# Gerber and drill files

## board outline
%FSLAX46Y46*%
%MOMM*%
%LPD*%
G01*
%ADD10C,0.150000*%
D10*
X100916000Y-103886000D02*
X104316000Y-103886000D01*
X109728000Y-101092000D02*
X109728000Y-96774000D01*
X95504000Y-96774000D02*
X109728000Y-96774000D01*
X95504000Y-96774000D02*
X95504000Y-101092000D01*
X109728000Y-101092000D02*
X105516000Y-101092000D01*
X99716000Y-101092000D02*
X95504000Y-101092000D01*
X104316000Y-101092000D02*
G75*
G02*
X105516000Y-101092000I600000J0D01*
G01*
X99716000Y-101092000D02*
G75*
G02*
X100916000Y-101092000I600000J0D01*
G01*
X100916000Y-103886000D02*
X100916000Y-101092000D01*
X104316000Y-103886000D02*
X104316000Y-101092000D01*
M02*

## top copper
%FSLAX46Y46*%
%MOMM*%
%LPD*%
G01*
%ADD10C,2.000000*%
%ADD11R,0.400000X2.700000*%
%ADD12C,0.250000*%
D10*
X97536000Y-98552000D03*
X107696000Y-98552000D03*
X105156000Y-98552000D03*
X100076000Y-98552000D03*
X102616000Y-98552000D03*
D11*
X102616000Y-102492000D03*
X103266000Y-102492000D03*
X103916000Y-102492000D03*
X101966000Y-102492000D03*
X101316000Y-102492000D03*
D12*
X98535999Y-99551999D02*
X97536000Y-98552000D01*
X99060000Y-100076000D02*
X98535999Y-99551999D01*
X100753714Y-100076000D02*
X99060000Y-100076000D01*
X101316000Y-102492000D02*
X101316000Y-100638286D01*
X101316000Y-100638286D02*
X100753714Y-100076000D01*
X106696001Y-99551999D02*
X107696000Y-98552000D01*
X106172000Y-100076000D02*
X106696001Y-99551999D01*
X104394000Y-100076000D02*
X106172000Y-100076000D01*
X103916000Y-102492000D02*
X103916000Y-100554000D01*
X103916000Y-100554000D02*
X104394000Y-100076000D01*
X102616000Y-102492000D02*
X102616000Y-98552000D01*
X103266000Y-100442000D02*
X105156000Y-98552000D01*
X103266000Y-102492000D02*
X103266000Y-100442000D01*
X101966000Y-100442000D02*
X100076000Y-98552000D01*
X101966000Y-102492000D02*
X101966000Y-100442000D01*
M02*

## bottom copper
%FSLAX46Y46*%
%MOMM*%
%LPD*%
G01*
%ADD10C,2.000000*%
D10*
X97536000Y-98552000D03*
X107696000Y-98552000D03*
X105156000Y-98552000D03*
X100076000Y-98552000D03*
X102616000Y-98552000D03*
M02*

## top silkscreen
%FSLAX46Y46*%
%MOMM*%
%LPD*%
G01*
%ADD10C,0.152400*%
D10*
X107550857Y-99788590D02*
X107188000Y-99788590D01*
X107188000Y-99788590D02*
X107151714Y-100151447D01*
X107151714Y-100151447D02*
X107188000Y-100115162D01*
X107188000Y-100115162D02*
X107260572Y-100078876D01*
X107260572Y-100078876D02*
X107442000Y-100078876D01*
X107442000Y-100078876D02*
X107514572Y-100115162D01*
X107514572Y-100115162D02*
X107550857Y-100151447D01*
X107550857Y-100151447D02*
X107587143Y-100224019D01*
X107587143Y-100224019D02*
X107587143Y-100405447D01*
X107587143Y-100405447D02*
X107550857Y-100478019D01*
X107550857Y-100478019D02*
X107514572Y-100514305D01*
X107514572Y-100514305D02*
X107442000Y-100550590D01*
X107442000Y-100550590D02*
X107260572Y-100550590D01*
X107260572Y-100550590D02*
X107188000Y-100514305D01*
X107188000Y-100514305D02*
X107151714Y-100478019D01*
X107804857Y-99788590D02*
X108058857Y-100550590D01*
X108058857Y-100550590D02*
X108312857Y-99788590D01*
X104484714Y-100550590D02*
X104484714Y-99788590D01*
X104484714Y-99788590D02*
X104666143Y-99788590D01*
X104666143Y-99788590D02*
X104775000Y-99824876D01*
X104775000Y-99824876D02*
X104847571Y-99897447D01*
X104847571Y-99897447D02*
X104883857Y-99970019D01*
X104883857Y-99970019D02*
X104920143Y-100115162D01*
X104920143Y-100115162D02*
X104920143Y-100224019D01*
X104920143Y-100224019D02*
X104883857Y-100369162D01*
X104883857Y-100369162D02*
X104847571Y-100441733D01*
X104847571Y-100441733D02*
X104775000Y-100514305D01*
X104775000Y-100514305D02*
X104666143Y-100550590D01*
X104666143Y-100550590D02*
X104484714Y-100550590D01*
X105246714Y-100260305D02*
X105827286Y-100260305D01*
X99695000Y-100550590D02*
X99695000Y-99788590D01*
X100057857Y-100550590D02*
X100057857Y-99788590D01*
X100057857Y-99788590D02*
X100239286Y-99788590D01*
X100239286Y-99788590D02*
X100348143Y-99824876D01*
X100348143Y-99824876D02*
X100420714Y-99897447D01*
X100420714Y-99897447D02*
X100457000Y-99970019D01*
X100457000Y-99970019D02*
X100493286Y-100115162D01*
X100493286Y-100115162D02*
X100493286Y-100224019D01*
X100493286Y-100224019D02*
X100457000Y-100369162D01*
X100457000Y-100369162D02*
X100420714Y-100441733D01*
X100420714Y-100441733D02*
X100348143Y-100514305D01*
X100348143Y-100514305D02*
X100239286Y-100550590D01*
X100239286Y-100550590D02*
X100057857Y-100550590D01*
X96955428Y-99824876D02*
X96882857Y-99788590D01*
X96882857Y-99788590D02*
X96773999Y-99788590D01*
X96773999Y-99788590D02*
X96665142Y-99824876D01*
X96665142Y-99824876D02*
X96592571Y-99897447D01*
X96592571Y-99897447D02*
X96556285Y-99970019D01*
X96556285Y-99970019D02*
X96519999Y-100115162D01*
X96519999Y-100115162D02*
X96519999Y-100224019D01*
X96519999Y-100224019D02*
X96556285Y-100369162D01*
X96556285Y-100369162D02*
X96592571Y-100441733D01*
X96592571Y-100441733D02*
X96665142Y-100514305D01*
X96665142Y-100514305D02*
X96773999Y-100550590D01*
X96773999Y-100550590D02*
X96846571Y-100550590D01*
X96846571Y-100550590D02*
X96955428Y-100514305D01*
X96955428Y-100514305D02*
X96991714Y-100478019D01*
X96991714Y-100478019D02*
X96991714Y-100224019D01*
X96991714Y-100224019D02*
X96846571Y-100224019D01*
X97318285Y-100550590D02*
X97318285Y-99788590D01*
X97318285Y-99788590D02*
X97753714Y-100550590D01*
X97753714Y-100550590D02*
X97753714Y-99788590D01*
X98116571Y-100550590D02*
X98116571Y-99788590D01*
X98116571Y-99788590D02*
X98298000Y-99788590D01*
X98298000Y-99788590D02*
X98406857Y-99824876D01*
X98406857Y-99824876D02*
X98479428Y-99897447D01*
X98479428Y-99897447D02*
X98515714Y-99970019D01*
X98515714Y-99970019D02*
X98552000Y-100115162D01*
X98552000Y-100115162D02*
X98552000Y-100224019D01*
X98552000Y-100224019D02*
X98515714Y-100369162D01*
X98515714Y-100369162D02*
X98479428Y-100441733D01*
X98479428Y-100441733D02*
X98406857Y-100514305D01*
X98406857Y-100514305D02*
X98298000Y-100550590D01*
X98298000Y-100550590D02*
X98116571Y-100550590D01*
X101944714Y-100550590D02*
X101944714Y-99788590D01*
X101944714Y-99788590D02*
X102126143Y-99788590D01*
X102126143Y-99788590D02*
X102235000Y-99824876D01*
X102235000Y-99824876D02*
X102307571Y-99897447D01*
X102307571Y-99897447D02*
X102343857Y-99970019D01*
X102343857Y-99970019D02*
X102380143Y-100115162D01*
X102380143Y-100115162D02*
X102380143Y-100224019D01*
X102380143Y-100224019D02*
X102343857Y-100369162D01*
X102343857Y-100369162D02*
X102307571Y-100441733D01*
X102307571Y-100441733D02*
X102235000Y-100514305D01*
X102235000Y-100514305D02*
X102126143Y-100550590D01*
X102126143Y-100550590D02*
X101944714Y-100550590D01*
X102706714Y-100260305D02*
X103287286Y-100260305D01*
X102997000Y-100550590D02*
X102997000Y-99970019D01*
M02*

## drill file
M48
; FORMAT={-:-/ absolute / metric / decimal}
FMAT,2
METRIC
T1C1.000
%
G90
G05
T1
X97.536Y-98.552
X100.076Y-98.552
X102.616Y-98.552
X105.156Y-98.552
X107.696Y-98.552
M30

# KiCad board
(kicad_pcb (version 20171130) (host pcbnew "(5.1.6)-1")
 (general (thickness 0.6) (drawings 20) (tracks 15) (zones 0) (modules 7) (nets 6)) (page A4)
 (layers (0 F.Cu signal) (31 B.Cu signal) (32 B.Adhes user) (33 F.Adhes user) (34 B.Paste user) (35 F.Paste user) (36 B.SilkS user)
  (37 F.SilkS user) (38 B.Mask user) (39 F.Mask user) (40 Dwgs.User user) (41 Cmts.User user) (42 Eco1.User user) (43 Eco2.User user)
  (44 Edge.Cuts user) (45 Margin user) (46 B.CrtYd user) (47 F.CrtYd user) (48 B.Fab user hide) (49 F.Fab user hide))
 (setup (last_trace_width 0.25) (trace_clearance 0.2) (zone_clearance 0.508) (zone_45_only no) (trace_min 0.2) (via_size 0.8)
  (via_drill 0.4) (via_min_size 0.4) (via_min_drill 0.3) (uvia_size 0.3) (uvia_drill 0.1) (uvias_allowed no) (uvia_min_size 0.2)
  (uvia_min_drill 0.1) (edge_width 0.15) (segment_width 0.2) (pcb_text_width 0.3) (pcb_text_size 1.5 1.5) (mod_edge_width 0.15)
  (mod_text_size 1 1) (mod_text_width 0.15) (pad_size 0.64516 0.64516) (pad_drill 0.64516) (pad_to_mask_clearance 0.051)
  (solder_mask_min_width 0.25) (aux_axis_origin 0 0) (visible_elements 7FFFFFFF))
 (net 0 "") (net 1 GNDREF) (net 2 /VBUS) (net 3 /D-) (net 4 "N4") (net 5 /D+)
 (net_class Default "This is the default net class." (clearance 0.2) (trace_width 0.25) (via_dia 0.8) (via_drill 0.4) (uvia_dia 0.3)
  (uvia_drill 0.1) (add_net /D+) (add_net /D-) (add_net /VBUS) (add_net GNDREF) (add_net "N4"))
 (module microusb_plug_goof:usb (layer B.Cu) (at 102.616 102.616)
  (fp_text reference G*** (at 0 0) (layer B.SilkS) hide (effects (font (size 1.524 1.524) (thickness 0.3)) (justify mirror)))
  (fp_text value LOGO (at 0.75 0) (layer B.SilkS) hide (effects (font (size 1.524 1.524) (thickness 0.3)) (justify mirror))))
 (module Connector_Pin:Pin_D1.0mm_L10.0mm (layer F.Cu) (at 97.536 98.552)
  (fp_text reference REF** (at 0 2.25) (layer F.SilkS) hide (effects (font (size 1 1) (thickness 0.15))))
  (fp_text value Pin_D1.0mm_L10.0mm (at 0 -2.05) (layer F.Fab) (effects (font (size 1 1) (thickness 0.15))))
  (pad 1 thru_hole circle (at 0 0) (size 2 2) (drill 1) (layers *.Cu *.Mask) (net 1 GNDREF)))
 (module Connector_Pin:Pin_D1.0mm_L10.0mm (layer F.Cu) (at 107.696 98.552)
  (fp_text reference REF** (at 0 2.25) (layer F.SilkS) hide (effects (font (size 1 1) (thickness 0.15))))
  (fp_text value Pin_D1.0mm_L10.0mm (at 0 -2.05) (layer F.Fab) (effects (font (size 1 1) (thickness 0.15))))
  (pad 1 thru_hole circle (at 0 0) (size 2 2) (drill 1) (layers *.Cu *.Mask) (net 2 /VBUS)))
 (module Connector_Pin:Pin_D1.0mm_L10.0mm (layer F.Cu) (at 105.156 98.552)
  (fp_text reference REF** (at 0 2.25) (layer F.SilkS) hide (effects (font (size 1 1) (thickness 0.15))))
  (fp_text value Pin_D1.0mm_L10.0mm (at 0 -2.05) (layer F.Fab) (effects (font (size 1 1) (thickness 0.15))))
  (pad 1 thru_hole circle (at 0 0) (size 2 2) (drill 1) (layers *.Cu *.Mask) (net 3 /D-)))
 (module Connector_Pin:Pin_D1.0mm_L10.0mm (layer F.Cu) (at 100.076 98.552)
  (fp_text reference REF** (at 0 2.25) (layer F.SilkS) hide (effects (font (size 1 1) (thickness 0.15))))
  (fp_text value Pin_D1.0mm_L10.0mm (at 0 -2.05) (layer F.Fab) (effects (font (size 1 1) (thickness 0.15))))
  (pad 1 thru_hole circle (at 0 0) (size 2 2) (drill 1) (layers *.Cu *.Mask) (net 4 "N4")))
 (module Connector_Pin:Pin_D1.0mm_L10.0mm (layer F.Cu) (at 102.616 98.552)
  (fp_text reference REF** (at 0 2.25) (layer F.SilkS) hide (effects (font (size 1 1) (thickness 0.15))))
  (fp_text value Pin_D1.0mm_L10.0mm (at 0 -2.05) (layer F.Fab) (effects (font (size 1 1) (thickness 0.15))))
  (pad 1 thru_hole circle (at 0 0) (size 2 2) (drill 1) (layers *.Cu *.Mask) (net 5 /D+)))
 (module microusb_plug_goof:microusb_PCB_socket (layer F.Cu) (at 102.616 102.492 180)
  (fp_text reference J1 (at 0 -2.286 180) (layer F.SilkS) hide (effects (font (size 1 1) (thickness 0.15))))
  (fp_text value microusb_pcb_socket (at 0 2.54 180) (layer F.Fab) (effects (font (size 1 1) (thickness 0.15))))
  (pad 3 smd rect (at 0 0 180) (size 0.4 2.7) (layers F.Cu F.Paste F.Mask) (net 5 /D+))
  (pad 2 smd rect (at -0.65 0 180) (size 0.4 2.7) (layers F.Cu F.Paste F.Mask) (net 3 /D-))
  (pad 1 smd rect (at -1.3 0 180) (size 0.4 2.7) (layers F.Cu F.Paste F.Mask) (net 2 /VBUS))
  (pad 4 smd rect (at 0.65 0 180) (size 0.4 2.7) (layers F.Cu F.Paste F.Mask) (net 4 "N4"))
  (pad 5 smd rect (at 1.3 0 180) (size 0.4 2.7) (layers F.Cu F.Paste F.Mask) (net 1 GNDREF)))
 (gr_line (start 100.916 103.886) (end 104.316 103.886) (layer Edge.Cuts) (width 0.15))
 (gr_line (start 109.728 101.092) (end 109.728 96.774) (layer Edge.Cuts) (width 0.15))
 (gr_line (start 95.504 96.774) (end 109.728 96.774) (layer Edge.Cuts) (width 0.15))
 (gr_line (start 95.504 96.774) (end 95.504 101.092) (layer Edge.Cuts) (width 0.15))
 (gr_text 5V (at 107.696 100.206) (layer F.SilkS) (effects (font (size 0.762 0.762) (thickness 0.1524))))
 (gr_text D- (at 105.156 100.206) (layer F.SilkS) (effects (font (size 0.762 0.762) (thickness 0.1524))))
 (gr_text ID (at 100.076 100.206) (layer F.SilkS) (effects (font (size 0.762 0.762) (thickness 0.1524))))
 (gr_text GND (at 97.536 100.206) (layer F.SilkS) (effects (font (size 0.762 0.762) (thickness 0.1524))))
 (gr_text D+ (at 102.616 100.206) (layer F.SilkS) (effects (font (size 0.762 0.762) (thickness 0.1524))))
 (gr_line (start 109.728 101.092) (end 105.516 101.092) (layer Edge.Cuts) (width 0.15))
 (gr_line (start 99.716 101.092) (end 95.504 101.092) (layer Edge.Cuts) (width 0.15))
 (gr_arc (start 104.916 101.092) (end 104.316 101.092) (angle 180) (layer Edge.Cuts) (width 0.15))
 (gr_arc (start 100.316 101.092) (end 100.916 101.092) (angle -180) (layer Edge.Cuts) (width 0.15))
 (gr_line (start 100.916 103.886) (end 100.916 101.092) (layer Edge.Cuts) (width 0.15))
 (gr_line (start 104.316 103.886) (end 104.316 101.092) (layer Edge.Cuts) (width 0.15))
 (segment (start 98.535999 99.551999) (end 97.536 98.552) (width 0.25) (layer F.Cu) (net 1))
 (segment (start 99.06 100.076) (end 98.535999 99.551999) (width 0.25) (layer F.Cu) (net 1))
 (segment (start 100.753714 100.076) (end 99.06 100.076) (width 0.25) (layer F.Cu) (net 1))
 (segment (start 101.316 102.492) (end 101.316 100.638286) (width 0.25) (layer F.Cu) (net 1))
 (segment (start 101.316 100.638286) (end 100.753714 100.076) (width 0.25) (layer F.Cu) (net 1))
 (segment (start 106.696001 99.551999) (end 107.696 98.552) (width 0.25) (layer F.Cu) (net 2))
 (segment (start 106.172 100.076) (end 106.696001 99.551999) (width 0.25) (layer F.Cu) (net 2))
 (segment (start 104.394 100.076) (end 106.172 100.076) (width 0.25) (layer F.Cu) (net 2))
 (segment (start 103.916 102.492) (end 103.916 100.554) (width 0.25) (layer F.Cu) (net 2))
 (segment (start 103.916 100.554) (end 104.394 100.076) (width 0.25) (layer F.Cu) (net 2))
 (segment (start 102.616 102.492) (end 102.616 98.552) (width 0.25) (layer F.Cu) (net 5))
 (segment (start 103.266 100.442) (end 105.156 98.552) (width 0.25) (layer F.Cu) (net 3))
 (segment (start 103.266 102.492) (end 103.266 100.442) (width 0.25) (layer F.Cu) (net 3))
 (segment (start 101.966 100.442) (end 100.076 98.552) (width 0.25) (layer F.Cu) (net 4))
 (segment (start 101.966 102.492) (end 101.966 100.442) (width 0.25) (layer F.Cu) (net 4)))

